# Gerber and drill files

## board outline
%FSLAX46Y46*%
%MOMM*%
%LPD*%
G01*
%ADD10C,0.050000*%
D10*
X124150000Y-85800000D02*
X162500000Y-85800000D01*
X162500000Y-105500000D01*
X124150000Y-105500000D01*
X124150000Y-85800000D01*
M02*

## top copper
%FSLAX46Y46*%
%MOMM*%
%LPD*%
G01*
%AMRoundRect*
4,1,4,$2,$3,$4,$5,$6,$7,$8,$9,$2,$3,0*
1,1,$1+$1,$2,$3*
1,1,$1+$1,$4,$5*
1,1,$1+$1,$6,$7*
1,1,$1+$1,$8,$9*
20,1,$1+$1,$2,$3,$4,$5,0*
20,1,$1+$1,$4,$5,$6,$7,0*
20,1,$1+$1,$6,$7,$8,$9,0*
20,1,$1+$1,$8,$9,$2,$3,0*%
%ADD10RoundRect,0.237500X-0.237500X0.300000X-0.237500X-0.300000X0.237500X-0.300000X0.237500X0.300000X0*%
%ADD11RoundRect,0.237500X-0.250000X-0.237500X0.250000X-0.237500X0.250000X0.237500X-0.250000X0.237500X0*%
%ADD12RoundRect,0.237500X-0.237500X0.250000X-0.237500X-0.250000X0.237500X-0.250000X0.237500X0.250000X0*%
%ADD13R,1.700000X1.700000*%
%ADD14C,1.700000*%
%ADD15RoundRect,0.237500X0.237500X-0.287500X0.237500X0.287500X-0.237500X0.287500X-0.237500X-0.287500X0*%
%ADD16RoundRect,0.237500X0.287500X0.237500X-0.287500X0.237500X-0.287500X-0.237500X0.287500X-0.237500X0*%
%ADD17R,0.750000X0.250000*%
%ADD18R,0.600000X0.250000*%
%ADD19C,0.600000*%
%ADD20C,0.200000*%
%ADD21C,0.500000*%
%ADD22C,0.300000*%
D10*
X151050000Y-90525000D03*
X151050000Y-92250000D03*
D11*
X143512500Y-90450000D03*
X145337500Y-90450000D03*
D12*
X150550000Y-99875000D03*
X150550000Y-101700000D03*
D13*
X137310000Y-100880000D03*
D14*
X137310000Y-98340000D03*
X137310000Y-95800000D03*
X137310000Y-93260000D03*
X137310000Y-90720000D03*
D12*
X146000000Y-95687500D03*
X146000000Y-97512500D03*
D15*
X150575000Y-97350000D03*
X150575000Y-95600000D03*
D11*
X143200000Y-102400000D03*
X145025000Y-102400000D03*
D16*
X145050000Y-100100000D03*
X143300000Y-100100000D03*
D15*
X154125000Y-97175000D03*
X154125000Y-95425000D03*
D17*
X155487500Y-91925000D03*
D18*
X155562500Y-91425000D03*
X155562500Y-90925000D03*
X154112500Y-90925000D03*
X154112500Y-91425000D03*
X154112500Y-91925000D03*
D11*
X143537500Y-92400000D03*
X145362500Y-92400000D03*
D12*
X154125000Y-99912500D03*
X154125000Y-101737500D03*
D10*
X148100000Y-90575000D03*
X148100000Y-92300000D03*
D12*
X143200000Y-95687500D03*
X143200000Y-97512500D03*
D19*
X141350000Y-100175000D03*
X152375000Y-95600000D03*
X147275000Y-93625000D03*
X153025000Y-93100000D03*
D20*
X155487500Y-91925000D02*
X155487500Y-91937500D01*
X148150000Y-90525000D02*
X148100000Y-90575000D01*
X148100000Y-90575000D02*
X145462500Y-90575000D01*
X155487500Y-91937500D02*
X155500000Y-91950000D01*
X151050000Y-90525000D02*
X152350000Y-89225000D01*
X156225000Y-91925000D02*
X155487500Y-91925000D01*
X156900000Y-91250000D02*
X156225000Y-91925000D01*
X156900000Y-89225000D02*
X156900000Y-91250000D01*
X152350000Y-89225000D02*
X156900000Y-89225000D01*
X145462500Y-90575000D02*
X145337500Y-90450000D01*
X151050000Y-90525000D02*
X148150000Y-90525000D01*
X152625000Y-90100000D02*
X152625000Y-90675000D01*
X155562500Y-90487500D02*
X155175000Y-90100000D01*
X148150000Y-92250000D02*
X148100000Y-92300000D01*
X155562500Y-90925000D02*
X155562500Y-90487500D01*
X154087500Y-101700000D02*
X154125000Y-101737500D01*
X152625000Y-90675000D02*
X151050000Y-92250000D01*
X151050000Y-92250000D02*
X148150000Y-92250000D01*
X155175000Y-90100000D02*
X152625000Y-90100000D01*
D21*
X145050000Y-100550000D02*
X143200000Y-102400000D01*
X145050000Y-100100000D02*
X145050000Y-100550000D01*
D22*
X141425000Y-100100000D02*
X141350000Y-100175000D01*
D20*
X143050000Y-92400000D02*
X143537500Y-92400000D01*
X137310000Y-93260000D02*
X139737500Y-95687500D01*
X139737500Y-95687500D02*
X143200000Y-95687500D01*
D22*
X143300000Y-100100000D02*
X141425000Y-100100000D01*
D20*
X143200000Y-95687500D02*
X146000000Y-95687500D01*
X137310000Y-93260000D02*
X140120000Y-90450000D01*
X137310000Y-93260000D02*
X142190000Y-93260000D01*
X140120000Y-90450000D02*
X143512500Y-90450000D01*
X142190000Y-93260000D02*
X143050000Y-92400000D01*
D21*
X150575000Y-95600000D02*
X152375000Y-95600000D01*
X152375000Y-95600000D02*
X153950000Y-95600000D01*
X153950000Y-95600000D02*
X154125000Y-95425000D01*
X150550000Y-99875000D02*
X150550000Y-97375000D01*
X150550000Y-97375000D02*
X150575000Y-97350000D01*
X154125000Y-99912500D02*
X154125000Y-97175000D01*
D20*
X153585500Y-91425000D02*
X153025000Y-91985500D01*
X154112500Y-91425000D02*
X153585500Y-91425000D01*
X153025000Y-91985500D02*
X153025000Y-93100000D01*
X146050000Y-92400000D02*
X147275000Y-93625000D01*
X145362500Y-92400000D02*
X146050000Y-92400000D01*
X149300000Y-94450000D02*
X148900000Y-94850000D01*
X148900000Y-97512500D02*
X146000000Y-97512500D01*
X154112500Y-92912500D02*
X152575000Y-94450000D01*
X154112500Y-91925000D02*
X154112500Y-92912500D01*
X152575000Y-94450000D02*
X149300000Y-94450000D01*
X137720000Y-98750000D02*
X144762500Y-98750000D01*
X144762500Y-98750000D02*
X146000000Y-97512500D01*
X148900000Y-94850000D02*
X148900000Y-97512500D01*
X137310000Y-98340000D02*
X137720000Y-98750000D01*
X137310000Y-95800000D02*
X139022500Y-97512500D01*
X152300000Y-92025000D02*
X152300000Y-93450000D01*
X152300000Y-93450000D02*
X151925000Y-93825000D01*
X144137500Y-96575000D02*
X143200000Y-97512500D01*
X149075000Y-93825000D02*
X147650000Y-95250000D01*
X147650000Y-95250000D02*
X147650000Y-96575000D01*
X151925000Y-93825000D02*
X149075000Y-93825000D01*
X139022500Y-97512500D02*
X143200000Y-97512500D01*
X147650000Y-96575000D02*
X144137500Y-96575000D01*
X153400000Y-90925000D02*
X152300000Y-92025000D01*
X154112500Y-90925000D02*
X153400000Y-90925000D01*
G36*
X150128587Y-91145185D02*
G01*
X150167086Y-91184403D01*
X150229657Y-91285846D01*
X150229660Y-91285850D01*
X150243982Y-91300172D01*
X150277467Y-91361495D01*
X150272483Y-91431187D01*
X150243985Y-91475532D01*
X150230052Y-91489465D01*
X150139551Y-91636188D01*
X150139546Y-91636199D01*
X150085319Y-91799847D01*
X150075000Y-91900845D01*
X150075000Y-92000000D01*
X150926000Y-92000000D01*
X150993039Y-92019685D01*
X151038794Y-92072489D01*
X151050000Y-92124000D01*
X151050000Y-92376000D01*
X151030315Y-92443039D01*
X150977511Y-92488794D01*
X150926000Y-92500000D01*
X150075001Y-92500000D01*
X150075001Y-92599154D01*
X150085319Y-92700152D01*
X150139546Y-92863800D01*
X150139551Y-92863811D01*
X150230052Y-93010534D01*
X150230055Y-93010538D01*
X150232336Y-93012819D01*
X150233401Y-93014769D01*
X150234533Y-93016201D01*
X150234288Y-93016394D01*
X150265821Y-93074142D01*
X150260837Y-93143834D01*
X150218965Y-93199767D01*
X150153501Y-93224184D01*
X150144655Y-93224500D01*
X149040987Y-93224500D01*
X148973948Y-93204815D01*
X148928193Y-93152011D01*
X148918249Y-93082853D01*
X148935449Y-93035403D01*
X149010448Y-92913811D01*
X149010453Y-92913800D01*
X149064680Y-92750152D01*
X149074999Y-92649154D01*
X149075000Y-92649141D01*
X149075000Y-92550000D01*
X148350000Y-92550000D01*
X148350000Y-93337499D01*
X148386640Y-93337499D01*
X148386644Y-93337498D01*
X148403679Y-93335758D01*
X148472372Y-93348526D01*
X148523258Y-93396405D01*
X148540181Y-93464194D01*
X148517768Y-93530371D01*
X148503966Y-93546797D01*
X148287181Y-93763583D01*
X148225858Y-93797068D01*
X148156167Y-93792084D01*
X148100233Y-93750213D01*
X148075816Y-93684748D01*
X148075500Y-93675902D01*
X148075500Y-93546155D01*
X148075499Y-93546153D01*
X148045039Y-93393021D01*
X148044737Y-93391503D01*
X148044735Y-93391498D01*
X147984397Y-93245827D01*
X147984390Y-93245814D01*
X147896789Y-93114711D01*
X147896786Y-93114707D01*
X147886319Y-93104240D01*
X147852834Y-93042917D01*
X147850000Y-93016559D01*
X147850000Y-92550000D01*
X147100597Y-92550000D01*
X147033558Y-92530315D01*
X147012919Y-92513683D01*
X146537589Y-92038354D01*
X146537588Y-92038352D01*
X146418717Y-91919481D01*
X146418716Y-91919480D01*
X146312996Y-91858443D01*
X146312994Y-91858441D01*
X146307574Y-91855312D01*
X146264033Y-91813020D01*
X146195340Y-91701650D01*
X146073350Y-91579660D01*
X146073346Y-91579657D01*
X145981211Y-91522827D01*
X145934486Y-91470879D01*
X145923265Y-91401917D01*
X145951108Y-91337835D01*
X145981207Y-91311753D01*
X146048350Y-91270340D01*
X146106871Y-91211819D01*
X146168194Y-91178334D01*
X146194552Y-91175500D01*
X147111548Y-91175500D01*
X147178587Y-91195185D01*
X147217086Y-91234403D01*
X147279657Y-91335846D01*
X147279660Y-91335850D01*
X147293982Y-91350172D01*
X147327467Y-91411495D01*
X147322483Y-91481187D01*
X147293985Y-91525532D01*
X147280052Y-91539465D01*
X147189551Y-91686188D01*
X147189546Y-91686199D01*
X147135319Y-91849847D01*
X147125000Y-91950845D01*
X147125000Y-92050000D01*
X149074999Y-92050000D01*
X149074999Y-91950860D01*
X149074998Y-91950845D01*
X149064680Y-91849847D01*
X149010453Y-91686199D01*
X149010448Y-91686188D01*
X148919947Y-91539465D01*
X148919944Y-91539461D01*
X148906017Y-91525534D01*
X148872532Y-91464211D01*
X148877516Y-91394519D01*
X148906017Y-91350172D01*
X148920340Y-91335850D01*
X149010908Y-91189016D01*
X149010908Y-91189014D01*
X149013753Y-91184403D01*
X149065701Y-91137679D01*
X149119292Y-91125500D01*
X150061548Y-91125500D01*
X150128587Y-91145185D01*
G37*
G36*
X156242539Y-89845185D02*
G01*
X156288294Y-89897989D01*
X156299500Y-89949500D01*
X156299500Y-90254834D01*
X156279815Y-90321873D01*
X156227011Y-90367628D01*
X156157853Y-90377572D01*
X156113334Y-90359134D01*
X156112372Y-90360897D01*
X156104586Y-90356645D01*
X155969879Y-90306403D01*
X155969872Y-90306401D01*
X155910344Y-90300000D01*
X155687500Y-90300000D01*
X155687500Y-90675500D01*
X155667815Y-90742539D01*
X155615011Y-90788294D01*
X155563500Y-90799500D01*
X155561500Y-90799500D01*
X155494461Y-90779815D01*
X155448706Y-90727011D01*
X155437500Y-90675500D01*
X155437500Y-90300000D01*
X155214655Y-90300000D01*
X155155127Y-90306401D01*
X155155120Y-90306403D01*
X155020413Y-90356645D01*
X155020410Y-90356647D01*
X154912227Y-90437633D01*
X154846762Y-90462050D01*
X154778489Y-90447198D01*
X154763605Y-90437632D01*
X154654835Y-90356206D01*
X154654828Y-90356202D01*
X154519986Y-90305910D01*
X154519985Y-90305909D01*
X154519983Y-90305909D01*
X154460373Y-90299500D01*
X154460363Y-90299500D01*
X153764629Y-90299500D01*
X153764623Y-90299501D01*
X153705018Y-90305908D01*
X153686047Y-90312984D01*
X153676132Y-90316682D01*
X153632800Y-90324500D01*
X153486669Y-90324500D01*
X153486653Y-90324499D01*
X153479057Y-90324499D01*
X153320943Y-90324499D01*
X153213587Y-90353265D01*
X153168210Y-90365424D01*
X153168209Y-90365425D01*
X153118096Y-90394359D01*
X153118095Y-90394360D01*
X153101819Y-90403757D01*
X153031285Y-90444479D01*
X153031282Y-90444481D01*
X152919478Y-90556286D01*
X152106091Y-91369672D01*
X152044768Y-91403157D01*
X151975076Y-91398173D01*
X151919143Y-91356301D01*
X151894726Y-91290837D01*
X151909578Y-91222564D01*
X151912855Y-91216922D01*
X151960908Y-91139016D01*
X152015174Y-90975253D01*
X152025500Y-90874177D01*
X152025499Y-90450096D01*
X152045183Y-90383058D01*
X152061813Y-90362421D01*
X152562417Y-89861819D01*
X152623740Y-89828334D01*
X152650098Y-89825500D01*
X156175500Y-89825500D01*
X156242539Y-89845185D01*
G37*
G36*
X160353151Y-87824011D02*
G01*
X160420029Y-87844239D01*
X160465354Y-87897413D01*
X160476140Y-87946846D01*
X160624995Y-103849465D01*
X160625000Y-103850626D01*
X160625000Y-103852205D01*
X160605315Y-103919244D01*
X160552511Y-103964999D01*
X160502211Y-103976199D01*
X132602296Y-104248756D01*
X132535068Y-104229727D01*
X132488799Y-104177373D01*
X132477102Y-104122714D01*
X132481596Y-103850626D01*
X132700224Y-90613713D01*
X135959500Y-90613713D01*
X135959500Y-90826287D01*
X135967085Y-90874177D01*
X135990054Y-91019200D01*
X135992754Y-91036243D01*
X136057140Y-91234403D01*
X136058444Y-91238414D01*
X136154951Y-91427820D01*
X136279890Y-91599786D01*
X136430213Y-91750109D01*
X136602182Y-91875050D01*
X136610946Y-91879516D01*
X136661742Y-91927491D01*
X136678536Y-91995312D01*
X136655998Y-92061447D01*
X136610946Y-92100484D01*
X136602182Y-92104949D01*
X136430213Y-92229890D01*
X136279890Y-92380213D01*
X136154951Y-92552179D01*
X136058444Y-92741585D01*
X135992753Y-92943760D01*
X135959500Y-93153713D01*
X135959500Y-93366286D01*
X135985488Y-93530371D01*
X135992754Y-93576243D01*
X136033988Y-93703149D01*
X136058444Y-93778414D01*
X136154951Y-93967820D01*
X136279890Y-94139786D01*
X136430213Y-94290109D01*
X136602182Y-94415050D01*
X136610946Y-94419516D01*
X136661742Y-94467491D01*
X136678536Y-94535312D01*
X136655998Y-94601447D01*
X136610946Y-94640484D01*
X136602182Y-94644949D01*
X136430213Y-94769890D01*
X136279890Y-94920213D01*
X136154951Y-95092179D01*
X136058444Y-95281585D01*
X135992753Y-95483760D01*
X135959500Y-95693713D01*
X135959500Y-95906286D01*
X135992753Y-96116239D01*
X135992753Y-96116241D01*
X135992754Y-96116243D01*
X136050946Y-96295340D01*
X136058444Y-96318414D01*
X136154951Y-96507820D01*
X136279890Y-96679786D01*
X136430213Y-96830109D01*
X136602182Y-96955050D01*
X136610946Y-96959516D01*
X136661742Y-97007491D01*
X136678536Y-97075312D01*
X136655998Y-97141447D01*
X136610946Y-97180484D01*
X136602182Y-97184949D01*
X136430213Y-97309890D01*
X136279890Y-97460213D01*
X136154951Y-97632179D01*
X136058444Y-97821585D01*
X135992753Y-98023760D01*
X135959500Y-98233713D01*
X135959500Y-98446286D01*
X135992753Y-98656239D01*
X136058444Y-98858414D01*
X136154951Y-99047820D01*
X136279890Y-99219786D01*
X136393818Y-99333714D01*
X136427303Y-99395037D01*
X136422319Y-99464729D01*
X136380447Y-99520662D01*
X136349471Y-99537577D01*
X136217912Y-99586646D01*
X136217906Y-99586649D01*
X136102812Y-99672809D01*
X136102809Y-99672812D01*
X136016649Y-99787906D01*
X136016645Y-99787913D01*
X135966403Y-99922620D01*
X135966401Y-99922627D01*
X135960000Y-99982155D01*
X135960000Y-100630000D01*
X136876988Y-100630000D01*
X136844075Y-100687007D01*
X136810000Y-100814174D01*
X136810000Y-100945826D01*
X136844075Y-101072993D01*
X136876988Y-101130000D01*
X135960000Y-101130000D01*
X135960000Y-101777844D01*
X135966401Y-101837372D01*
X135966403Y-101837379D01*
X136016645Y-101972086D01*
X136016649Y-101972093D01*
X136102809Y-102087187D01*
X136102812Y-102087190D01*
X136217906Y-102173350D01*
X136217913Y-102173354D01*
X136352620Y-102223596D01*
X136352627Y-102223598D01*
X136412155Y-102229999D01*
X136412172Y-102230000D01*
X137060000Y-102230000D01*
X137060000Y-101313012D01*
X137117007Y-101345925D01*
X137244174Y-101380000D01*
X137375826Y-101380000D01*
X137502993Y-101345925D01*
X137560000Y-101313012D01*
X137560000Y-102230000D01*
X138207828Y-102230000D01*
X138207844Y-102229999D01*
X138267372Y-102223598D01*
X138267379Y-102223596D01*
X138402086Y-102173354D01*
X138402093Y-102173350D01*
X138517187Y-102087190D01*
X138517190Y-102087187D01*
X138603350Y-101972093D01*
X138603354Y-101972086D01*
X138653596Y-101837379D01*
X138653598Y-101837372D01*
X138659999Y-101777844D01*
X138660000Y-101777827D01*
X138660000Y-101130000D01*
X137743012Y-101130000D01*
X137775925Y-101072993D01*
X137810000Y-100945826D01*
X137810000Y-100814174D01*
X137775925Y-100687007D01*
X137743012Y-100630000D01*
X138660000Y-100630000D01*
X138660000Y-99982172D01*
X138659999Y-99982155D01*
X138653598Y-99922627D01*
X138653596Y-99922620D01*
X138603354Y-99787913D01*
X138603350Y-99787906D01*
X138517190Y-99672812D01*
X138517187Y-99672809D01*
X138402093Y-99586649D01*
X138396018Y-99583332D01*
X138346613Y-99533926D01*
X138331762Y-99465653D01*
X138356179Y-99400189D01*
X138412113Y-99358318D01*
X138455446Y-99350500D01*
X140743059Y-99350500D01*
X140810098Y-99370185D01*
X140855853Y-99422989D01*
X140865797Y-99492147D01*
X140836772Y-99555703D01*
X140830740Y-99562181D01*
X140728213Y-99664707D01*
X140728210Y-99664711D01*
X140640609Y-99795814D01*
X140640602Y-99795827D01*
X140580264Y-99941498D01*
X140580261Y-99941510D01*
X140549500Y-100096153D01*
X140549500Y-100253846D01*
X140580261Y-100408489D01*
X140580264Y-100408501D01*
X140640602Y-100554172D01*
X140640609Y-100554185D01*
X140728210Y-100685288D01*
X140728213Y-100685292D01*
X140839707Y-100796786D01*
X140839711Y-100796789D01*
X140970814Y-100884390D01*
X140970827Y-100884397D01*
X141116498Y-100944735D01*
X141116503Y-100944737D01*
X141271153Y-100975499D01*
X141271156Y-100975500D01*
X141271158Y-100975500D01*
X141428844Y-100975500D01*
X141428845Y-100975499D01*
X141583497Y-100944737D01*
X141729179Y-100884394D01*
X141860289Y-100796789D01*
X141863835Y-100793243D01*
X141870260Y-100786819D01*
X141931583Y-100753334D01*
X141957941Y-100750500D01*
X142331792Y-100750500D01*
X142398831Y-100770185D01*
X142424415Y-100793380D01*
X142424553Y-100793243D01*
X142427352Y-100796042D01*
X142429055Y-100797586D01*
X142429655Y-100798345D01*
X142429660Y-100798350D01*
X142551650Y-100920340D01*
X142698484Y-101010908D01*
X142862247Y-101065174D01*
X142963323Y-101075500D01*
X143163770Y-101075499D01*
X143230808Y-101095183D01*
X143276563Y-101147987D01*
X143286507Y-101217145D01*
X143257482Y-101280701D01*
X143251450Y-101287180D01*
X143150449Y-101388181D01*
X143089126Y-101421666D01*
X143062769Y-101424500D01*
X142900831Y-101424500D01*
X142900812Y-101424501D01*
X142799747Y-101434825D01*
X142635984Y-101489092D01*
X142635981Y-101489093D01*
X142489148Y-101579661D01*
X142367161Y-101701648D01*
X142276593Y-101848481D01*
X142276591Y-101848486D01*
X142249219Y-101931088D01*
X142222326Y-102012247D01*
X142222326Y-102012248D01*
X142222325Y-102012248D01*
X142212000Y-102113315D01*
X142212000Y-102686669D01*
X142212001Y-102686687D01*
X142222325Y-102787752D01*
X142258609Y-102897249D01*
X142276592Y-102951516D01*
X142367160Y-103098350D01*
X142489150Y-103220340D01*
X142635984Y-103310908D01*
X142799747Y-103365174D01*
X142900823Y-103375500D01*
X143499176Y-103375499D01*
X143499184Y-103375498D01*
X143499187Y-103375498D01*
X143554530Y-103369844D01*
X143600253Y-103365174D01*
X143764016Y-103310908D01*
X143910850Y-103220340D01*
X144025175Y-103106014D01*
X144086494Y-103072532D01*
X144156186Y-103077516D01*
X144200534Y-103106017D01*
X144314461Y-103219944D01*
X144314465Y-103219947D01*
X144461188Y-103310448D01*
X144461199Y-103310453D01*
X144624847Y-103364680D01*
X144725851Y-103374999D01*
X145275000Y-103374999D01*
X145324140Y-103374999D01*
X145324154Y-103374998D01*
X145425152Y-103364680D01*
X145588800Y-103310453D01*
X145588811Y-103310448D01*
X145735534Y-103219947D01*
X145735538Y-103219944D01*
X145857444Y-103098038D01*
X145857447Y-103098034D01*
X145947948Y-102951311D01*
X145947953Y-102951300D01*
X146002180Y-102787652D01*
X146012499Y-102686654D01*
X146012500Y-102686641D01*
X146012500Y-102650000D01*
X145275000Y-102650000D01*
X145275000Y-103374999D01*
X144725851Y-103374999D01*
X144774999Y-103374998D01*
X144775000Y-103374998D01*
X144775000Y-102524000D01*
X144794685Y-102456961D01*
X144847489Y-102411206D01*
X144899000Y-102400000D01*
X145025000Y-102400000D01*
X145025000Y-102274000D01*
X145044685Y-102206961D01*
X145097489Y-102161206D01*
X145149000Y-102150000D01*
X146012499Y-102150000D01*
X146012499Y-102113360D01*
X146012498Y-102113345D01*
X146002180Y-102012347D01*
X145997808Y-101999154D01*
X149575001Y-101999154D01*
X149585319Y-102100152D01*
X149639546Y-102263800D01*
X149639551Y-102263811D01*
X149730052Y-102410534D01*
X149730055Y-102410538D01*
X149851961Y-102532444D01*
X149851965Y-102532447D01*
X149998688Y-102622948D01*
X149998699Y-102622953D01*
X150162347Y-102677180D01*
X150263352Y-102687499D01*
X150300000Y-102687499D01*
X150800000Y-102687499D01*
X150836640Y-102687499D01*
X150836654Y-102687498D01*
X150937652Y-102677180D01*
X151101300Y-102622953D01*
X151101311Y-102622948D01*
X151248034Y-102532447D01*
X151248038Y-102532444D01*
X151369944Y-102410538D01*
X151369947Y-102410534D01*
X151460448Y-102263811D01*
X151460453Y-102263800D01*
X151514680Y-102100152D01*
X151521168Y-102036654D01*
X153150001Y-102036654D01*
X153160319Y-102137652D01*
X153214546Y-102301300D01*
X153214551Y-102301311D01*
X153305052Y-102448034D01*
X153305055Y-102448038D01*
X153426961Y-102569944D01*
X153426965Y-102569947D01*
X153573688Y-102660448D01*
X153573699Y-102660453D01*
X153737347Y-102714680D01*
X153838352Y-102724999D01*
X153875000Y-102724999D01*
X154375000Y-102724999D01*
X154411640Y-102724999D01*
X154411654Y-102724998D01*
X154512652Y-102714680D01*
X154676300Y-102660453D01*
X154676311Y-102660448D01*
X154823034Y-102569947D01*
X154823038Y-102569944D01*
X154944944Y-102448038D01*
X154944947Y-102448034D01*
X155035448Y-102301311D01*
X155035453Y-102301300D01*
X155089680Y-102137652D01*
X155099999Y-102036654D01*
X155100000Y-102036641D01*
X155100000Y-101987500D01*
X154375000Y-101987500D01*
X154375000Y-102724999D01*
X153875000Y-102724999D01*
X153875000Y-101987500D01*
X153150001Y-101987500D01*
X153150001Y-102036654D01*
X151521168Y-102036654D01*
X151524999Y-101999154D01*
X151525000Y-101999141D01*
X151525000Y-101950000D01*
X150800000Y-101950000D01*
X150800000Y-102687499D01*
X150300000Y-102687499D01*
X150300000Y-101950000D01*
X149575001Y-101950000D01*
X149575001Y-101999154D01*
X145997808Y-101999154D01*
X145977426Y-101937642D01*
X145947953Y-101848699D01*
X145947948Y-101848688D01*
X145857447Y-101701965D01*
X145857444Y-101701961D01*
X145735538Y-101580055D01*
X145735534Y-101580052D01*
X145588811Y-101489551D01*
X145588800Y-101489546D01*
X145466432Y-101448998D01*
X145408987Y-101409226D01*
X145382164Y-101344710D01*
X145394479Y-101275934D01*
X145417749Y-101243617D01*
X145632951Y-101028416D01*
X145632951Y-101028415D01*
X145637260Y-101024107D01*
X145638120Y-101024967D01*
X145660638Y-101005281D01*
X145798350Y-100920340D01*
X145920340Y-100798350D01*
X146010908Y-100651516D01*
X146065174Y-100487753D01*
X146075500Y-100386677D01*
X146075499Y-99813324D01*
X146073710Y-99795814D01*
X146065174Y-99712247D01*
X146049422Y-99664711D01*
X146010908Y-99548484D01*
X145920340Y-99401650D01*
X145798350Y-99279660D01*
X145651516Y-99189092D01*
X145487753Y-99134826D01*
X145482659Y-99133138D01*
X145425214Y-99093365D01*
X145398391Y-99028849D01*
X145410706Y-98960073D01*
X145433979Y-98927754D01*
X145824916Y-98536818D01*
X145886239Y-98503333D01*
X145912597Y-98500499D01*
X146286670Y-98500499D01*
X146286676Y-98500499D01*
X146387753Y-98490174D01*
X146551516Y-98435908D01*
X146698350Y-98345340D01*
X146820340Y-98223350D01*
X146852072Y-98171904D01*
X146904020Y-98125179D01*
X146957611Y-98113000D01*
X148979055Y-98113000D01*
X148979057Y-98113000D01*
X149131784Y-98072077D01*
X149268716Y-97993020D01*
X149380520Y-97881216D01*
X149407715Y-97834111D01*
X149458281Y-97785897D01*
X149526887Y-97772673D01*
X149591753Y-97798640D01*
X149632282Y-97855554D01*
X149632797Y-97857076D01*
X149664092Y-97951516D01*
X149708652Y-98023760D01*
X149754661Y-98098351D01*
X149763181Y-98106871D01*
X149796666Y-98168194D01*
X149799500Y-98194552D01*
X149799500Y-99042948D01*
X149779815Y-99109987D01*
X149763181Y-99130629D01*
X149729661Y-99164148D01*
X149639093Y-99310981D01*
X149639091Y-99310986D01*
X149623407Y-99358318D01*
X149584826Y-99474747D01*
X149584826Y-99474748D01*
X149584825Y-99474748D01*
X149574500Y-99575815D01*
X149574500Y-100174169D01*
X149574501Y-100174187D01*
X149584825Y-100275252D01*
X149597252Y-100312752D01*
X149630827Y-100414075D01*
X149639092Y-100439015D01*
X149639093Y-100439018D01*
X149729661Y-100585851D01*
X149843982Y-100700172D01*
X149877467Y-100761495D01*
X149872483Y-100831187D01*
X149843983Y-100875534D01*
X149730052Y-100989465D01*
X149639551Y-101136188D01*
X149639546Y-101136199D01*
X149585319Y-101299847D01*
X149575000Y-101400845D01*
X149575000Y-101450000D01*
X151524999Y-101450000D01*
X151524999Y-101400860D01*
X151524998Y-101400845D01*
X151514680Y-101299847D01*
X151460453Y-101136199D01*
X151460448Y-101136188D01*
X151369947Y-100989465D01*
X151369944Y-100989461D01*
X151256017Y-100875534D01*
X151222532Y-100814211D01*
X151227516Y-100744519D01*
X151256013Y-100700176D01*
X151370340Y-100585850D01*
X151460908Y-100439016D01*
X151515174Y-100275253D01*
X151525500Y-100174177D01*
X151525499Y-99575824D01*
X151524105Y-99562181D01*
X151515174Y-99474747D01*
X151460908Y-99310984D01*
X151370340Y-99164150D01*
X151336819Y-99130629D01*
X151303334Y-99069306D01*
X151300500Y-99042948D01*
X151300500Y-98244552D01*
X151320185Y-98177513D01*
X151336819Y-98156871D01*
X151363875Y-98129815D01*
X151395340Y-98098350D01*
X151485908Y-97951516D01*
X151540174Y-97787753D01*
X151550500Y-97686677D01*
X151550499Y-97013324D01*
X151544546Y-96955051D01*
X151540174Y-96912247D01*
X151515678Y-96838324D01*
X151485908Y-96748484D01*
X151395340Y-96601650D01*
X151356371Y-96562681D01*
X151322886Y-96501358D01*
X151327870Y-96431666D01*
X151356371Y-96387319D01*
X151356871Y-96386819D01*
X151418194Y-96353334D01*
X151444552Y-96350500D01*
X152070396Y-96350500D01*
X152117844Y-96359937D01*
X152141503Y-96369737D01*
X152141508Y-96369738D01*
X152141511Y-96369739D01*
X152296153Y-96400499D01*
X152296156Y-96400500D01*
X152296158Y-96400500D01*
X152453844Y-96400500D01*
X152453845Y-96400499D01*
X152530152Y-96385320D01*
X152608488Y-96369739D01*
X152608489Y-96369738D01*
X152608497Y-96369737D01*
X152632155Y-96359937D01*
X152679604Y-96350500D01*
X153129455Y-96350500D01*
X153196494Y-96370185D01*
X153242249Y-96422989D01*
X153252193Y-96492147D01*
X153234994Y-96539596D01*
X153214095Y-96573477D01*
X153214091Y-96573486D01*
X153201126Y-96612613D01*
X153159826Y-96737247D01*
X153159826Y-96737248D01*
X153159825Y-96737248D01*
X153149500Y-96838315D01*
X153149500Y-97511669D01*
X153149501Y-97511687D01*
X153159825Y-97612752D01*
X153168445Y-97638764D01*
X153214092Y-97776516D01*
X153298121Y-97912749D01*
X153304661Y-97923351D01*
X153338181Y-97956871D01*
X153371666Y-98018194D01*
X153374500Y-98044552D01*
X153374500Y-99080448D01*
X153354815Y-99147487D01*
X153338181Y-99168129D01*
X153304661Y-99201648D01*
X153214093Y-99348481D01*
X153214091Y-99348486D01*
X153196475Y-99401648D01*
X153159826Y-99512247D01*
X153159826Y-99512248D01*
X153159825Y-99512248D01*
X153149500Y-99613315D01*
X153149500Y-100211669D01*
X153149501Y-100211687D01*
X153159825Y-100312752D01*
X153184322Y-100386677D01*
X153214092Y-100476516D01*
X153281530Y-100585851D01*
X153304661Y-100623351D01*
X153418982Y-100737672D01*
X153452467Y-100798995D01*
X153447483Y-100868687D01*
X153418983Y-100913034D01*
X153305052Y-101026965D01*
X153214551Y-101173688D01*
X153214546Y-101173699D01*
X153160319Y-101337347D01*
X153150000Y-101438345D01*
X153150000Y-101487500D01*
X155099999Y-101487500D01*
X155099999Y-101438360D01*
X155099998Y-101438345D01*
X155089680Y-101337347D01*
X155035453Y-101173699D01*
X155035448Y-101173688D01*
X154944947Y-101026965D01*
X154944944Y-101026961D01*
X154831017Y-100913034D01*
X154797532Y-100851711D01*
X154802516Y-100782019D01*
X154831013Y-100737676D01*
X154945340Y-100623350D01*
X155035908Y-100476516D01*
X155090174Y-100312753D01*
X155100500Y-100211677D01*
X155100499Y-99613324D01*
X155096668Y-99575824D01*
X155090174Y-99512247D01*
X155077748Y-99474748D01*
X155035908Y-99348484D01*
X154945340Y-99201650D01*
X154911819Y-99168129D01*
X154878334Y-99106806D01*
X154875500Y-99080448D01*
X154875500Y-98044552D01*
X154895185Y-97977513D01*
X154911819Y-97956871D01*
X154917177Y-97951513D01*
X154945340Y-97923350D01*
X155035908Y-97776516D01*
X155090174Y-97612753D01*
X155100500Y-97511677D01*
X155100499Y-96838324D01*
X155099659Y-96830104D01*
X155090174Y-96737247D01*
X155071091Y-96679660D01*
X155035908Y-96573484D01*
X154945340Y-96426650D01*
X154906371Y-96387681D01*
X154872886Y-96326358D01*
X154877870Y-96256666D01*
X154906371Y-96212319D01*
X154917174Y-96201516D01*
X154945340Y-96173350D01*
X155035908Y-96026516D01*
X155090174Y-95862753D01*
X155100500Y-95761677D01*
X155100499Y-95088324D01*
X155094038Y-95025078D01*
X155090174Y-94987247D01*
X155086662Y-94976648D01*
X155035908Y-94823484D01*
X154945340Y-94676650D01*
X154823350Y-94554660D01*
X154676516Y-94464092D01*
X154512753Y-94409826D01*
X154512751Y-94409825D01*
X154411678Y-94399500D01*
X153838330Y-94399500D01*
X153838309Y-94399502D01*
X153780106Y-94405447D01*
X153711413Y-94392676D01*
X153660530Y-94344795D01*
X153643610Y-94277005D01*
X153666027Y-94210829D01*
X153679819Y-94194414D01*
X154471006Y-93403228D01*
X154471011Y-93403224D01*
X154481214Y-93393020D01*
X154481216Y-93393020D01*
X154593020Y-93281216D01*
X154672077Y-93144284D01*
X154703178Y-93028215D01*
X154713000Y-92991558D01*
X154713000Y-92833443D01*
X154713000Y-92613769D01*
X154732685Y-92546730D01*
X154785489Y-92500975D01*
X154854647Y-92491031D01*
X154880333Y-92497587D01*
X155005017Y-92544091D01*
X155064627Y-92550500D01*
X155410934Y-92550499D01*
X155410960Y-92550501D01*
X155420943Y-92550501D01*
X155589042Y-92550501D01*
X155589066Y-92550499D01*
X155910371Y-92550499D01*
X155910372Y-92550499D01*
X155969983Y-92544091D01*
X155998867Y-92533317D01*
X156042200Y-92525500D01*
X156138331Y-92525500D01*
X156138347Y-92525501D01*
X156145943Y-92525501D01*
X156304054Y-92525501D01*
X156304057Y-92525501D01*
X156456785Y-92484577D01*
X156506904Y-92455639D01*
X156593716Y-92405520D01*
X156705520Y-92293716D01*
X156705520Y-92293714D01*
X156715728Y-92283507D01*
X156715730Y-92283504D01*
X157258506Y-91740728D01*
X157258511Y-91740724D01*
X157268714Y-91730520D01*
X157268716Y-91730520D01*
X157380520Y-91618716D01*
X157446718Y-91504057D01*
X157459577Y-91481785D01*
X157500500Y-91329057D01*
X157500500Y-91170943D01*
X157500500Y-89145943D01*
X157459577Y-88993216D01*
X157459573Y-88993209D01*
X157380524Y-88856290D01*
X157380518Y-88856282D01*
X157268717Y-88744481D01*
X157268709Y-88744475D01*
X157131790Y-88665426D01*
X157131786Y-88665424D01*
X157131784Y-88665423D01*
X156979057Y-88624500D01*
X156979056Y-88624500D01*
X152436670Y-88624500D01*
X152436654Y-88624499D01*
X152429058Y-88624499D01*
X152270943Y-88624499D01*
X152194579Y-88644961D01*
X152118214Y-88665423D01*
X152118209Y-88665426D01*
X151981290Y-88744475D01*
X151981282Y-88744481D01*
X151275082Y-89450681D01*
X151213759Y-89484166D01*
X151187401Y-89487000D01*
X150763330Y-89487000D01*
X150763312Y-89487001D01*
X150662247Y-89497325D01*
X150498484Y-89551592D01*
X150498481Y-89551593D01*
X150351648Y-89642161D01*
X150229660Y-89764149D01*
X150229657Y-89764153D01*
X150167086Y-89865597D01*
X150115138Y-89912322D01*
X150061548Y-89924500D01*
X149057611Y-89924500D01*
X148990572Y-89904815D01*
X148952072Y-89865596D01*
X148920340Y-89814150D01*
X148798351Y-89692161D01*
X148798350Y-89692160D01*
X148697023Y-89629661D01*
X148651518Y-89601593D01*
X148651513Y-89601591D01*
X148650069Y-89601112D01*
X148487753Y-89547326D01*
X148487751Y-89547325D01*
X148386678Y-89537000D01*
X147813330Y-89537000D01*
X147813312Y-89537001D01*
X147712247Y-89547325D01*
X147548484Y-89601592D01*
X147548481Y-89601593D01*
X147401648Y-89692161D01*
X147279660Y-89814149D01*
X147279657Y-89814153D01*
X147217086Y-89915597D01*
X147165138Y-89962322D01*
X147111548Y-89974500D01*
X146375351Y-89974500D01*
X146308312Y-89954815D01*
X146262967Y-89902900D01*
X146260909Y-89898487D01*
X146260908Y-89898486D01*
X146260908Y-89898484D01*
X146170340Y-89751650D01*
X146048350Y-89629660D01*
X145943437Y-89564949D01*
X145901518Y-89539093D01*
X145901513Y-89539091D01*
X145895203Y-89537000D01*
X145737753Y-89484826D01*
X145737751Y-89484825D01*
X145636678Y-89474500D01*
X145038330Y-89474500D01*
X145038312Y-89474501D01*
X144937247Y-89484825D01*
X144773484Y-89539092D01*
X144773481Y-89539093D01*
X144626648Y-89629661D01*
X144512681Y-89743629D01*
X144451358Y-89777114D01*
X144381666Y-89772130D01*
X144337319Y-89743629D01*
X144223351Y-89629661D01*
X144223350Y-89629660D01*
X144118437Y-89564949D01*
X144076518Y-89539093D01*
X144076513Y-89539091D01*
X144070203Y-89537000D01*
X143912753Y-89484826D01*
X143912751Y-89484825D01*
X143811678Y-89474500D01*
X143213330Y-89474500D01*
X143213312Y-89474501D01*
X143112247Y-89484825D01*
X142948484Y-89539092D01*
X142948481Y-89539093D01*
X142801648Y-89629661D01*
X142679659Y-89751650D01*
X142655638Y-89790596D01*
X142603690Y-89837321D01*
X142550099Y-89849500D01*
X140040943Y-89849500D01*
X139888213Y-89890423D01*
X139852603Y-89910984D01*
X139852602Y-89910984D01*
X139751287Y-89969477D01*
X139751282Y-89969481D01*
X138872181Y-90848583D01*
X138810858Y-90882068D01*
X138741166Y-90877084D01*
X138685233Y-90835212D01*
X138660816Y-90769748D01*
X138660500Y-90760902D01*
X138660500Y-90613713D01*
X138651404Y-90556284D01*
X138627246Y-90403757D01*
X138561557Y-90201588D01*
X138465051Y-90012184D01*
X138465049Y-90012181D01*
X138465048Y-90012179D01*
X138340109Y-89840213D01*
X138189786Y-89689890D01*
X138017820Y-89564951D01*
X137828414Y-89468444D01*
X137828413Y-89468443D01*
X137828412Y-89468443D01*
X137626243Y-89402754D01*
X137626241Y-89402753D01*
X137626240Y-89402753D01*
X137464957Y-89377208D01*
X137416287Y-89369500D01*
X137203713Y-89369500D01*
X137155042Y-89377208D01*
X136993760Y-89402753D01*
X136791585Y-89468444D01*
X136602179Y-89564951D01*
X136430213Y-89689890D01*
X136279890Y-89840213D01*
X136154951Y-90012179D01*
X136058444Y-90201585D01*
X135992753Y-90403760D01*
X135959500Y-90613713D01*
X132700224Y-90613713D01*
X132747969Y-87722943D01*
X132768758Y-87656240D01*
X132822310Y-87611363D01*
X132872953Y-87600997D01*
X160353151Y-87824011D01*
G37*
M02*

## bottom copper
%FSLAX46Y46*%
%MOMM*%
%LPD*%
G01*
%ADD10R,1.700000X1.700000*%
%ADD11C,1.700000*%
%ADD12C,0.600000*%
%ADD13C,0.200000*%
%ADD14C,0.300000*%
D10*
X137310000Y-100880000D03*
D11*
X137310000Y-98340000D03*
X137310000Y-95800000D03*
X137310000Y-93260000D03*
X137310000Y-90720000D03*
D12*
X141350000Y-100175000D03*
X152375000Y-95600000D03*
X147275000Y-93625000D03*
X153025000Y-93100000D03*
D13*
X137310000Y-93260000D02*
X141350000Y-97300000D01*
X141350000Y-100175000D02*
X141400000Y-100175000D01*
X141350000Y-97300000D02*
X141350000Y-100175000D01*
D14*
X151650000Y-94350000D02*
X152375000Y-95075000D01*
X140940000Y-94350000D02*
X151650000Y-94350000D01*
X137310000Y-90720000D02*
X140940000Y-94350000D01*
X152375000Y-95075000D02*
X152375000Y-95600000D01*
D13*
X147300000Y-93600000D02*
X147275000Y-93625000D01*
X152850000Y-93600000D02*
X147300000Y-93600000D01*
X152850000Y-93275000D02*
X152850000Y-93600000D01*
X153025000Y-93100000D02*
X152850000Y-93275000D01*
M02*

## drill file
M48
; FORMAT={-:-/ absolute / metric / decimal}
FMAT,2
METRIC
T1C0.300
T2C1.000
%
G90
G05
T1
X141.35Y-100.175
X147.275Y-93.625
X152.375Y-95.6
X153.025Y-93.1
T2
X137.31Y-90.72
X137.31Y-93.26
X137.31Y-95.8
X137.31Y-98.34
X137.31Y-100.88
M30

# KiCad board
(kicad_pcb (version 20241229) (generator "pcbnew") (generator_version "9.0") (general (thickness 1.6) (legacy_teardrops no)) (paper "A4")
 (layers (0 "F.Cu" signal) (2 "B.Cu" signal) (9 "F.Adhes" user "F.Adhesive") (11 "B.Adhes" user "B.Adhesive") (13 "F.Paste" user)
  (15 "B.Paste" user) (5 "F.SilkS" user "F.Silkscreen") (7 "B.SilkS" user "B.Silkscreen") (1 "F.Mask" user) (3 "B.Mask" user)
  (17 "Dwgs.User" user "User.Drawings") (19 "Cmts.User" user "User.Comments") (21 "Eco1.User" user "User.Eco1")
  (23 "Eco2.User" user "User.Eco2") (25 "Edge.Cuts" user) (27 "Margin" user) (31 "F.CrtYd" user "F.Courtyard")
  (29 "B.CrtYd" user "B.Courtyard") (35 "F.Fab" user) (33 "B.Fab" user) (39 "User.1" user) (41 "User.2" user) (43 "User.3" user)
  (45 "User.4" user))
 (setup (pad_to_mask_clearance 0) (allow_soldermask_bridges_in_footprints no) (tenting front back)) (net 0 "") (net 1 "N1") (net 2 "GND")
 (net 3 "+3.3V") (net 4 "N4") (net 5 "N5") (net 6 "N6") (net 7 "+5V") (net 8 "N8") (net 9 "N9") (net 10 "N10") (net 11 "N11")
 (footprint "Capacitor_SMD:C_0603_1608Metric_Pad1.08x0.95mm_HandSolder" (layer "F.Cu") (at 151.05 91.3875 -90)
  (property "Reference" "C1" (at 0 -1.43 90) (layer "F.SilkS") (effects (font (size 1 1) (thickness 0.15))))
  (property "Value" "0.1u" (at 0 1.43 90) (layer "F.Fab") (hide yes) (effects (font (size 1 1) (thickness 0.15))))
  (pad "1" smd roundrect (at -0.8625 0 270) (size 1.075 0.95) (layers "F.Cu" "F.Mask" "F.Paste") (roundrect_rratio 0.25) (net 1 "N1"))
  (pad "2" smd roundrect (at 0.8625 0 270) (size 1.075 0.95) (layers "F.Cu" "F.Mask" "F.Paste") (roundrect_rratio 0.25) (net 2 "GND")))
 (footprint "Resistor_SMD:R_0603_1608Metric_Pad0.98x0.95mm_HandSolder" (layer "F.Cu") (at 144.425 90.45)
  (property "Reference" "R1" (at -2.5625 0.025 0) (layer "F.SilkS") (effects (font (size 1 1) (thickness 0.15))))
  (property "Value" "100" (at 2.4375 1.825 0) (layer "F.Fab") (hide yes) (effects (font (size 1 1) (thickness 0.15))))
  (pad "1" smd roundrect (at -0.9125 0) (size 0.975 0.95) (layers "F.Cu" "F.Mask" "F.Paste") (roundrect_rratio 0.25) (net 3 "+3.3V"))
  (pad "2" smd roundrect (at 0.9125 0) (size 0.975 0.95) (layers "F.Cu" "F.Mask" "F.Paste") (roundrect_rratio 0.25) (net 1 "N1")))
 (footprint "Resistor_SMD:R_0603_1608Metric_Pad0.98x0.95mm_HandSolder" (layer "F.Cu") (at 150.55 100.7875 -90)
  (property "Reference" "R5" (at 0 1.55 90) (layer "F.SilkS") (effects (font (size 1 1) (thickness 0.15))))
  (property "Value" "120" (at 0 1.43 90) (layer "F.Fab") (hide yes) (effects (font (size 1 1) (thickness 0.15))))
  (pad "1" smd roundrect (at -0.9125 0 270) (size 0.975 0.95) (layers "F.Cu" "F.Mask" "F.Paste") (roundrect_rratio 0.25) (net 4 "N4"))
  (pad "2" smd roundrect (at 0.9125 0 270) (size 0.975 0.95) (layers "F.Cu" "F.Mask" "F.Paste") (roundrect_rratio 0.25) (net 2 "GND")))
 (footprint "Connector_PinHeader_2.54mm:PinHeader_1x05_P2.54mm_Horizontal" (layer "F.Cu") (at 137.31 100.88 180)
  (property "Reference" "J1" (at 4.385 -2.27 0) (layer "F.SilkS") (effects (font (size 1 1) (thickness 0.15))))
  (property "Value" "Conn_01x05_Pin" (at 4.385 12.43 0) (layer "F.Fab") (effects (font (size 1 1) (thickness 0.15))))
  (pad "1" thru_hole rect (at 0 0 180) (size 1.7 1.7) (drill 1) (layers "*.Cu" "*.Mask") (remove_unused_layers no) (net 2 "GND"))
  (pad "2" thru_hole circle (at 0 2.54 180) (size 1.7 1.7) (drill 1) (layers "*.Cu" "*.Mask") (remove_unused_layers no) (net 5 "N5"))
  (pad "3" thru_hole circle (at 0 5.08 180) (size 1.7 1.7) (drill 1) (layers "*.Cu" "*.Mask") (remove_unused_layers no) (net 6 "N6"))
  (pad "4" thru_hole circle (at 0 7.62 180) (size 1.7 1.7) (drill 1) (layers "*.Cu" "*.Mask") (remove_unused_layers no) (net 3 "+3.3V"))
  (pad "5" thru_hole circle (at 0 10.16 180) (size 1.7 1.7) (drill 1) (layers "*.Cu" "*.Mask") (remove_unused_layers no) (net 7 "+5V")))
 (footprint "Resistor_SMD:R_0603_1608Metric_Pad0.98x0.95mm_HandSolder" (layer "F.Cu") (at 146 96.6 -90)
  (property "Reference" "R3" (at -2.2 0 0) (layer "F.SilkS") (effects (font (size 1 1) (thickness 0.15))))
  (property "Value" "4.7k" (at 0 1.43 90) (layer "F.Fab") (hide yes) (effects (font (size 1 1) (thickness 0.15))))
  (pad "1" smd roundrect (at -0.9125 0 270) (size 0.975 0.95) (layers "F.Cu" "F.Mask" "F.Paste") (roundrect_rratio 0.25) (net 3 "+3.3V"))
  (pad "2" smd roundrect (at 0.9125 0 270) (size 0.975 0.95) (layers "F.Cu" "F.Mask" "F.Paste") (roundrect_rratio 0.25) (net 5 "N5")))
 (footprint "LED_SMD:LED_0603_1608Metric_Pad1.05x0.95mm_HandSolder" (layer "F.Cu") (at 150.575 96.475 90)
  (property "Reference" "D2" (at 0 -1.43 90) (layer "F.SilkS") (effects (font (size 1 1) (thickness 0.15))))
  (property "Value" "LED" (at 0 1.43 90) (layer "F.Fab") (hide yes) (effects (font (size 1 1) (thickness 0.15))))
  (pad "1" smd roundrect (at -0.875 0 90) (size 1.05 0.95) (layers "F.Cu" "F.Mask" "F.Paste") (roundrect_rratio 0.25) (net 4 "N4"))
  (pad "2" smd roundrect (at 0.875 0 90) (size 1.05 0.95) (layers "F.Cu" "F.Mask" "F.Paste") (roundrect_rratio 0.25) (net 7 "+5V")))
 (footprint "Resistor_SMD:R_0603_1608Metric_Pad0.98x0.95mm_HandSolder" (layer "F.Cu") (at 144.1125 102.4)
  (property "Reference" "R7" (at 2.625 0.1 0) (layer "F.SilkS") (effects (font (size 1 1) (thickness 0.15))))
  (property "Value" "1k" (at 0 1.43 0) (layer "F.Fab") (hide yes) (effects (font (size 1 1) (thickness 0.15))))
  (pad "1" smd roundrect (at -0.9125 0) (size 0.975 0.95) (layers "F.Cu" "F.Mask" "F.Paste") (roundrect_rratio 0.25) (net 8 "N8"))
  (pad "2" smd roundrect (at 0.9125 0) (size 0.975 0.95) (layers "F.Cu" "F.Mask" "F.Paste") (roundrect_rratio 0.25) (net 2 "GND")))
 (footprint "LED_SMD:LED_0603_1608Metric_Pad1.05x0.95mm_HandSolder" (layer "F.Cu") (at 144.175 100.1 180)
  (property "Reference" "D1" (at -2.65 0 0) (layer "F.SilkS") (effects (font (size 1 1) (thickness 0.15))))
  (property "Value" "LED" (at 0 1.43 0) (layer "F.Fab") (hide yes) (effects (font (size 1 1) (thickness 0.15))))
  (pad "1" smd roundrect (at -0.875 0 180) (size 1.05 0.95) (layers "F.Cu" "F.Mask" "F.Paste") (roundrect_rratio 0.25) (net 8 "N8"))
  (pad "2" smd roundrect (at 0.875 0 180) (size 1.05 0.95) (layers "F.Cu" "F.Mask" "F.Paste") (roundrect_rratio 0.25) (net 3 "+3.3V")))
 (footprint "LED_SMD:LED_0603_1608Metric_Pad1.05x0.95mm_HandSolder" (layer "F.Cu") (at 154.125 96.3 90)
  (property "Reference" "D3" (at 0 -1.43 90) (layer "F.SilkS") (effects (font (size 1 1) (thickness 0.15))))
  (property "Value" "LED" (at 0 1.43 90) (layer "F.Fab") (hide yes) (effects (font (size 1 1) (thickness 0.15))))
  (pad "1" smd roundrect (at -0.875 0 90) (size 1.05 0.95) (layers "F.Cu" "F.Mask" "F.Paste") (roundrect_rratio 0.25) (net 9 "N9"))
  (pad "2" smd roundrect (at 0.875 0 90) (size 1.05 0.95) (layers "F.Cu" "F.Mask" "F.Paste") (roundrect_rratio 0.25) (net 7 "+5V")))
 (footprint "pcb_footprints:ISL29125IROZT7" (layer "F.Cu") (at 154.8375 91.425 180)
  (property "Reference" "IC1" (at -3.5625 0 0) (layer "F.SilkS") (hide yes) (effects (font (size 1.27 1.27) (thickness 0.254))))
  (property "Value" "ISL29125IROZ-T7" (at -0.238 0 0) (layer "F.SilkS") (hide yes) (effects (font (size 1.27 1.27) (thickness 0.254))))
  (pad "1" smd rect (at -0.65 -0.5 270) (size 0.25 0.75) (layers "F.Cu" "F.Mask" "F.Paste") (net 1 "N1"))
  (pad "2" smd rect (at -0.725 0 270) (size 0.25 0.6) (layers "F.Cu" "F.Mask" "F.Paste") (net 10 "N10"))
  (pad "3" smd rect (at -0.725 0.5 270) (size 0.25 0.6) (layers "F.Cu" "F.Mask" "F.Paste") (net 2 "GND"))
  (pad "4" smd rect (at 0.725 0.5 270) (size 0.25 0.6) (layers "F.Cu" "F.Mask" "F.Paste") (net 6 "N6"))
  (pad "5" smd rect (at 0.725 0 270) (size 0.25 0.6) (layers "F.Cu" "F.Mask" "F.Paste") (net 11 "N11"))
  (pad "6" smd rect (at 0.725 -0.5 270) (size 0.25 0.6) (layers "F.Cu" "F.Mask" "F.Paste") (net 5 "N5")))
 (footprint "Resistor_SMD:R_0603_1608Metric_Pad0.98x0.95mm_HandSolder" (layer "F.Cu") (at 144.45 92.4)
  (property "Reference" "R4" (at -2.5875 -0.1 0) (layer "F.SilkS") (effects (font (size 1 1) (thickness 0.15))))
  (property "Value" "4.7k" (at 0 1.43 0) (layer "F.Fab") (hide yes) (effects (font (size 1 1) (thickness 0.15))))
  (pad "1" smd roundrect (at -0.9125 0) (size 0.975 0.95) (layers "F.Cu" "F.Mask" "F.Paste") (roundrect_rratio 0.25) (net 3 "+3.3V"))
  (pad "2" smd roundrect (at 0.9125 0) (size 0.975 0.95) (layers "F.Cu" "F.Mask" "F.Paste") (roundrect_rratio 0.25) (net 11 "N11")))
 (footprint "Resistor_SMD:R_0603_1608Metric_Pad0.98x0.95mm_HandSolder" (layer "F.Cu") (at 154.125 100.825 -90)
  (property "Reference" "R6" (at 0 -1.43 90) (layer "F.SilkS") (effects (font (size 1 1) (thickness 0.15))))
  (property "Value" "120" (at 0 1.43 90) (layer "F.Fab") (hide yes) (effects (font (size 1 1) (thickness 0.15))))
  (pad "1" smd roundrect (at -0.9125 0 270) (size 0.975 0.95) (layers "F.Cu" "F.Mask" "F.Paste") (roundrect_rratio 0.25) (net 9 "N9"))
  (pad "2" smd roundrect (at 0.9125 0 270) (size 0.975 0.95) (layers "F.Cu" "F.Mask" "F.Paste") (roundrect_rratio 0.25) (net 2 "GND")))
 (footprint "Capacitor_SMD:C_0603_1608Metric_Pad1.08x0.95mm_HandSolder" (layer "F.Cu") (at 148.1 91.4375 -90)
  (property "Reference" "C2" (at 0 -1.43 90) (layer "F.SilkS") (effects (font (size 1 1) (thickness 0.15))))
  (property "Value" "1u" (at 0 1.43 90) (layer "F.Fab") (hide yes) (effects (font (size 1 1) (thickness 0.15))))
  (pad "1" smd roundrect (at -0.8625 0 270) (size 1.075 0.95) (layers "F.Cu" "F.Mask" "F.Paste") (roundrect_rratio 0.25) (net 1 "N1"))
  (pad "2" smd roundrect (at 0.8625 0 270) (size 1.075 0.95) (layers "F.Cu" "F.Mask" "F.Paste") (roundrect_rratio 0.25) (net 2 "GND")))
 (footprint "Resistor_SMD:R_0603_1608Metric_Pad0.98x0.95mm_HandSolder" (layer "F.Cu") (at 143.2 96.6 -90)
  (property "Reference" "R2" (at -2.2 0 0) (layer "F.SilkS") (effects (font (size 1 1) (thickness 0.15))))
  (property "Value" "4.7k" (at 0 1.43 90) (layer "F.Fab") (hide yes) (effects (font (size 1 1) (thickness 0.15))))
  (pad "1" smd roundrect (at -0.9125 0 270) (size 0.975 0.95) (layers "F.Cu" "F.Mask" "F.Paste") (roundrect_rratio 0.25) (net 3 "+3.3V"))
  (pad "2" smd roundrect (at 0.9125 0 270) (size 0.975 0.95) (layers "F.Cu" "F.Mask" "F.Paste") (roundrect_rratio 0.25) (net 6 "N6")))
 (gr_rect (start 124.15 85.8) (end 162.5 105.5) (stroke (width 0.05) (type default)) (fill no) (layer "Edge.Cuts"))
 (segment (start 155.4875 91.925) (end 155.4875 91.9375) (width 0.2) (layer "F.Cu") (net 1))
 (segment (start 148.15 90.525) (end 148.1 90.575) (width 0.2) (layer "F.Cu") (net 1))
 (segment (start 148.1 90.575) (end 145.4625 90.575) (width 0.2) (layer "F.Cu") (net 1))
 (segment (start 155.4875 91.9375) (end 155.5 91.95) (width 0.2) (layer "F.Cu") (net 1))
 (segment (start 151.05 90.525) (end 152.35 89.225) (width 0.2) (layer "F.Cu") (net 1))
 (segment (start 156.225 91.925) (end 155.4875 91.925) (width 0.2) (layer "F.Cu") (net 1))
 (segment (start 156.9 91.25) (end 156.225 91.925) (width 0.2) (layer "F.Cu") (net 1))
 (segment (start 156.9 89.225) (end 156.9 91.25) (width 0.2) (layer "F.Cu") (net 1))
 (segment (start 152.35 89.225) (end 156.9 89.225) (width 0.2) (layer "F.Cu") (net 1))
 (segment (start 145.4625 90.575) (end 145.3375 90.45) (width 0.2) (layer "F.Cu") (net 1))
 (segment (start 151.05 90.525) (end 148.15 90.525) (width 0.2) (layer "F.Cu") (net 1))
 (segment (start 152.625 90.1) (end 152.625 90.675) (width 0.2) (layer "F.Cu") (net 2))
 (segment (start 155.5625 90.4875) (end 155.175 90.1) (width 0.2) (layer "F.Cu") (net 2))
 (segment (start 148.15 92.25) (end 148.1 92.3) (width 0.2) (layer "F.Cu") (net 2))
 (segment (start 155.5625 90.925) (end 155.5625 90.4875) (width 0.2) (layer "F.Cu") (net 2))
 (segment (start 154.0875 101.7) (end 154.125 101.7375) (width 0.2) (layer "F.Cu") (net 2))
 (segment (start 152.625 90.675) (end 151.05 92.25) (width 0.2) (layer "F.Cu") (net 2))
 (segment (start 151.05 92.25) (end 148.15 92.25) (width 0.2) (layer "F.Cu") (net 2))
 (segment (start 155.175 90.1) (end 152.625 90.1) (width 0.2) (layer "F.Cu") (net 2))
 (segment (start 145.05 100.55) (end 143.2 102.4) (width 0.5) (layer "F.Cu") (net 8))
 (segment (start 145.05 100.1) (end 145.05 100.55) (width 0.5) (layer "F.Cu") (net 8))
 (segment (start 141.425 100.1) (end 141.35 100.175) (width 0.3) (layer "F.Cu") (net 3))
 (segment (start 143.05 92.4) (end 143.5375 92.4) (width 0.2) (layer "F.Cu") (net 3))
 (segment (start 137.31 93.26) (end 139.7375 95.6875) (width 0.2) (layer "F.Cu") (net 3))
 (segment (start 139.7375 95.6875) (end 143.2 95.6875) (width 0.2) (layer "F.Cu") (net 3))
 (segment (start 143.3 100.1) (end 141.425 100.1) (width 0.3) (layer "F.Cu") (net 3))
 (segment (start 143.2 95.6875) (end 146 95.6875) (width 0.2) (layer "F.Cu") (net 3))
 (segment (start 137.31 93.26) (end 140.12 90.45) (width 0.2) (layer "F.Cu") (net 3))
 (segment (start 137.31 93.26) (end 142.19 93.26) (width 0.2) (layer "F.Cu") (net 3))
 (segment (start 140.12 90.45) (end 143.5125 90.45) (width 0.2) (layer "F.Cu") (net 3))
 (segment (start 142.19 93.26) (end 143.05 92.4) (width 0.2) (layer "F.Cu") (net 3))
 (via (at 141.35 100.175) (size 0.6) (drill 0.3) (layers "F.Cu" "B.Cu") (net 3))
 (segment (start 137.31 93.26) (end 141.35 97.3) (width 0.2) (layer "B.Cu") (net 3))
 (segment (start 141.35 100.175) (end 141.4 100.175) (width 0.2) (layer "B.Cu") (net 3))
 (segment (start 141.35 97.3) (end 141.35 100.175) (width 0.2) (layer "B.Cu") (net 3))
 (segment (start 150.575 95.6) (end 152.375 95.6) (width 0.5) (layer "F.Cu") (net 7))
 (segment (start 152.375 95.6) (end 153.95 95.6) (width 0.5) (layer "F.Cu") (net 7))
 (segment (start 153.95 95.6) (end 154.125 95.425) (width 0.5) (layer "F.Cu") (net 7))
 (via (at 152.375 95.6) (size 0.6) (drill 0.3) (layers "F.Cu" "B.Cu") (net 7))
 (segment (start 151.65 94.35) (end 152.375 95.075) (width 0.3) (layer "B.Cu") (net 7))
 (segment (start 140.94 94.35) (end 151.65 94.35) (width 0.3) (layer "B.Cu") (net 7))
 (segment (start 137.31 90.72) (end 140.94 94.35) (width 0.3) (layer "B.Cu") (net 7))
 (segment (start 152.375 95.075) (end 152.375 95.6) (width 0.3) (layer "B.Cu") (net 7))
 (segment (start 150.55 99.875) (end 150.55 97.375) (width 0.5) (layer "F.Cu") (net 4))
 (segment (start 150.55 97.375) (end 150.575 97.35) (width 0.5) (layer "F.Cu") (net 4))
 (segment (start 154.125 99.9125) (end 154.125 97.175) (width 0.5) (layer "F.Cu") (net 9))
 (segment (start 153.5855 91.425) (end 153.025 91.9855) (width 0.2) (layer "F.Cu") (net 11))
 (segment (start 154.1125 91.425) (end 153.5855 91.425) (width 0.2) (layer "F.Cu") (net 11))
 (segment (start 153.025 91.9855) (end 153.025 93.1) (width 0.2) (layer "F.Cu") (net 11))
 (segment (start 146.05 92.4) (end 147.275 93.625) (width 0.2) (layer "F.Cu") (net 11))
 (segment (start 145.3625 92.4) (end 146.05 92.4) (width 0.2) (layer "F.Cu") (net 11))
 (via (at 147.275 93.625) (size 0.6) (drill 0.3) (layers "F.Cu" "B.Cu") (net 11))
 (via (at 153.025 93.1) (size 0.6) (drill 0.3) (layers "F.Cu" "B.Cu") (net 11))
 (segment (start 147.3 93.6) (end 147.275 93.625) (width 0.2) (layer "B.Cu") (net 11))
 (segment (start 152.85 93.6) (end 147.3 93.6) (width 0.2) (layer "B.Cu") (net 11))
 (segment (start 152.85 93.275) (end 152.85 93.6) (width 0.2) (layer "B.Cu") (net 11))
 (segment (start 153.025 93.1) (end 152.85 93.275) (width 0.2) (layer "B.Cu") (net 11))
 (segment (start 149.3 94.45) (end 148.9 94.85) (width 0.2) (layer "F.Cu") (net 5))
 (segment (start 148.9 97.5125) (end 146 97.5125) (width 0.2) (layer "F.Cu") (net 5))
 (segment (start 154.1125 92.9125) (end 152.575 94.45) (width 0.2) (layer "F.Cu") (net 5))
 (segment (start 154.1125 91.925) (end 154.1125 92.9125) (width 0.2) (layer "F.Cu") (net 5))
 (segment (start 152.575 94.45) (end 149.3 94.45) (width 0.2) (layer "F.Cu") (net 5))
 (segment (start 137.72 98.75) (end 144.7625 98.75) (width 0.2) (layer "F.Cu") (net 5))
 (segment (start 144.7625 98.75) (end 146 97.5125) (width 0.2) (layer "F.Cu") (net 5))
 (segment (start 148.9 94.85) (end 148.9 97.5125) (width 0.2) (layer "F.Cu") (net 5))
 (segment (start 137.31 98.34) (end 137.72 98.75) (width 0.2) (layer "F.Cu") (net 5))
 (segment (start 137.31 95.8) (end 139.0225 97.5125) (width 0.2) (layer "F.Cu") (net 6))
 (segment (start 152.3 92.025) (end 152.3 93.45) (width 0.2) (layer "F.Cu") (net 6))
 (segment (start 152.3 93.45) (end 151.925 93.825) (width 0.2) (layer "F.Cu") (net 6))
 (segment (start 144.1375 96.575) (end 143.2 97.5125) (width 0.2) (layer "F.Cu") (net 6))
 (segment (start 149.075 93.825) (end 147.65 95.25) (width 0.2) (layer "F.Cu") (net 6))
 (segment (start 147.65 95.25) (end 147.65 96.575) (width 0.2) (layer "F.Cu") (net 6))
 (segment (start 151.925 93.825) (end 149.075 93.825) (width 0.2) (layer "F.Cu") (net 6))
 (segment (start 139.0225 97.5125) (end 143.2 97.5125) (width 0.2) (layer "F.Cu") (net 6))
 (segment (start 147.65 96.575) (end 144.1375 96.575) (width 0.2) (layer "F.Cu") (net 6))
 (segment (start 153.4 90.925) (end 152.3 92.025) (width 0.2) (layer "F.Cu") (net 6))
 (segment (start 154.1125 90.925) (end 153.4 90.925) (width 0.2) (layer "F.Cu") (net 6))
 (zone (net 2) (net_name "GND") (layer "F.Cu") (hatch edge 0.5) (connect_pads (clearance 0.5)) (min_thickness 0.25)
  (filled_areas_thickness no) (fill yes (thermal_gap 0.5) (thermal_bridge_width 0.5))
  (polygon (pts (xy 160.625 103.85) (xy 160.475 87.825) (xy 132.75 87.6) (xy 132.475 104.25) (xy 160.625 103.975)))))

